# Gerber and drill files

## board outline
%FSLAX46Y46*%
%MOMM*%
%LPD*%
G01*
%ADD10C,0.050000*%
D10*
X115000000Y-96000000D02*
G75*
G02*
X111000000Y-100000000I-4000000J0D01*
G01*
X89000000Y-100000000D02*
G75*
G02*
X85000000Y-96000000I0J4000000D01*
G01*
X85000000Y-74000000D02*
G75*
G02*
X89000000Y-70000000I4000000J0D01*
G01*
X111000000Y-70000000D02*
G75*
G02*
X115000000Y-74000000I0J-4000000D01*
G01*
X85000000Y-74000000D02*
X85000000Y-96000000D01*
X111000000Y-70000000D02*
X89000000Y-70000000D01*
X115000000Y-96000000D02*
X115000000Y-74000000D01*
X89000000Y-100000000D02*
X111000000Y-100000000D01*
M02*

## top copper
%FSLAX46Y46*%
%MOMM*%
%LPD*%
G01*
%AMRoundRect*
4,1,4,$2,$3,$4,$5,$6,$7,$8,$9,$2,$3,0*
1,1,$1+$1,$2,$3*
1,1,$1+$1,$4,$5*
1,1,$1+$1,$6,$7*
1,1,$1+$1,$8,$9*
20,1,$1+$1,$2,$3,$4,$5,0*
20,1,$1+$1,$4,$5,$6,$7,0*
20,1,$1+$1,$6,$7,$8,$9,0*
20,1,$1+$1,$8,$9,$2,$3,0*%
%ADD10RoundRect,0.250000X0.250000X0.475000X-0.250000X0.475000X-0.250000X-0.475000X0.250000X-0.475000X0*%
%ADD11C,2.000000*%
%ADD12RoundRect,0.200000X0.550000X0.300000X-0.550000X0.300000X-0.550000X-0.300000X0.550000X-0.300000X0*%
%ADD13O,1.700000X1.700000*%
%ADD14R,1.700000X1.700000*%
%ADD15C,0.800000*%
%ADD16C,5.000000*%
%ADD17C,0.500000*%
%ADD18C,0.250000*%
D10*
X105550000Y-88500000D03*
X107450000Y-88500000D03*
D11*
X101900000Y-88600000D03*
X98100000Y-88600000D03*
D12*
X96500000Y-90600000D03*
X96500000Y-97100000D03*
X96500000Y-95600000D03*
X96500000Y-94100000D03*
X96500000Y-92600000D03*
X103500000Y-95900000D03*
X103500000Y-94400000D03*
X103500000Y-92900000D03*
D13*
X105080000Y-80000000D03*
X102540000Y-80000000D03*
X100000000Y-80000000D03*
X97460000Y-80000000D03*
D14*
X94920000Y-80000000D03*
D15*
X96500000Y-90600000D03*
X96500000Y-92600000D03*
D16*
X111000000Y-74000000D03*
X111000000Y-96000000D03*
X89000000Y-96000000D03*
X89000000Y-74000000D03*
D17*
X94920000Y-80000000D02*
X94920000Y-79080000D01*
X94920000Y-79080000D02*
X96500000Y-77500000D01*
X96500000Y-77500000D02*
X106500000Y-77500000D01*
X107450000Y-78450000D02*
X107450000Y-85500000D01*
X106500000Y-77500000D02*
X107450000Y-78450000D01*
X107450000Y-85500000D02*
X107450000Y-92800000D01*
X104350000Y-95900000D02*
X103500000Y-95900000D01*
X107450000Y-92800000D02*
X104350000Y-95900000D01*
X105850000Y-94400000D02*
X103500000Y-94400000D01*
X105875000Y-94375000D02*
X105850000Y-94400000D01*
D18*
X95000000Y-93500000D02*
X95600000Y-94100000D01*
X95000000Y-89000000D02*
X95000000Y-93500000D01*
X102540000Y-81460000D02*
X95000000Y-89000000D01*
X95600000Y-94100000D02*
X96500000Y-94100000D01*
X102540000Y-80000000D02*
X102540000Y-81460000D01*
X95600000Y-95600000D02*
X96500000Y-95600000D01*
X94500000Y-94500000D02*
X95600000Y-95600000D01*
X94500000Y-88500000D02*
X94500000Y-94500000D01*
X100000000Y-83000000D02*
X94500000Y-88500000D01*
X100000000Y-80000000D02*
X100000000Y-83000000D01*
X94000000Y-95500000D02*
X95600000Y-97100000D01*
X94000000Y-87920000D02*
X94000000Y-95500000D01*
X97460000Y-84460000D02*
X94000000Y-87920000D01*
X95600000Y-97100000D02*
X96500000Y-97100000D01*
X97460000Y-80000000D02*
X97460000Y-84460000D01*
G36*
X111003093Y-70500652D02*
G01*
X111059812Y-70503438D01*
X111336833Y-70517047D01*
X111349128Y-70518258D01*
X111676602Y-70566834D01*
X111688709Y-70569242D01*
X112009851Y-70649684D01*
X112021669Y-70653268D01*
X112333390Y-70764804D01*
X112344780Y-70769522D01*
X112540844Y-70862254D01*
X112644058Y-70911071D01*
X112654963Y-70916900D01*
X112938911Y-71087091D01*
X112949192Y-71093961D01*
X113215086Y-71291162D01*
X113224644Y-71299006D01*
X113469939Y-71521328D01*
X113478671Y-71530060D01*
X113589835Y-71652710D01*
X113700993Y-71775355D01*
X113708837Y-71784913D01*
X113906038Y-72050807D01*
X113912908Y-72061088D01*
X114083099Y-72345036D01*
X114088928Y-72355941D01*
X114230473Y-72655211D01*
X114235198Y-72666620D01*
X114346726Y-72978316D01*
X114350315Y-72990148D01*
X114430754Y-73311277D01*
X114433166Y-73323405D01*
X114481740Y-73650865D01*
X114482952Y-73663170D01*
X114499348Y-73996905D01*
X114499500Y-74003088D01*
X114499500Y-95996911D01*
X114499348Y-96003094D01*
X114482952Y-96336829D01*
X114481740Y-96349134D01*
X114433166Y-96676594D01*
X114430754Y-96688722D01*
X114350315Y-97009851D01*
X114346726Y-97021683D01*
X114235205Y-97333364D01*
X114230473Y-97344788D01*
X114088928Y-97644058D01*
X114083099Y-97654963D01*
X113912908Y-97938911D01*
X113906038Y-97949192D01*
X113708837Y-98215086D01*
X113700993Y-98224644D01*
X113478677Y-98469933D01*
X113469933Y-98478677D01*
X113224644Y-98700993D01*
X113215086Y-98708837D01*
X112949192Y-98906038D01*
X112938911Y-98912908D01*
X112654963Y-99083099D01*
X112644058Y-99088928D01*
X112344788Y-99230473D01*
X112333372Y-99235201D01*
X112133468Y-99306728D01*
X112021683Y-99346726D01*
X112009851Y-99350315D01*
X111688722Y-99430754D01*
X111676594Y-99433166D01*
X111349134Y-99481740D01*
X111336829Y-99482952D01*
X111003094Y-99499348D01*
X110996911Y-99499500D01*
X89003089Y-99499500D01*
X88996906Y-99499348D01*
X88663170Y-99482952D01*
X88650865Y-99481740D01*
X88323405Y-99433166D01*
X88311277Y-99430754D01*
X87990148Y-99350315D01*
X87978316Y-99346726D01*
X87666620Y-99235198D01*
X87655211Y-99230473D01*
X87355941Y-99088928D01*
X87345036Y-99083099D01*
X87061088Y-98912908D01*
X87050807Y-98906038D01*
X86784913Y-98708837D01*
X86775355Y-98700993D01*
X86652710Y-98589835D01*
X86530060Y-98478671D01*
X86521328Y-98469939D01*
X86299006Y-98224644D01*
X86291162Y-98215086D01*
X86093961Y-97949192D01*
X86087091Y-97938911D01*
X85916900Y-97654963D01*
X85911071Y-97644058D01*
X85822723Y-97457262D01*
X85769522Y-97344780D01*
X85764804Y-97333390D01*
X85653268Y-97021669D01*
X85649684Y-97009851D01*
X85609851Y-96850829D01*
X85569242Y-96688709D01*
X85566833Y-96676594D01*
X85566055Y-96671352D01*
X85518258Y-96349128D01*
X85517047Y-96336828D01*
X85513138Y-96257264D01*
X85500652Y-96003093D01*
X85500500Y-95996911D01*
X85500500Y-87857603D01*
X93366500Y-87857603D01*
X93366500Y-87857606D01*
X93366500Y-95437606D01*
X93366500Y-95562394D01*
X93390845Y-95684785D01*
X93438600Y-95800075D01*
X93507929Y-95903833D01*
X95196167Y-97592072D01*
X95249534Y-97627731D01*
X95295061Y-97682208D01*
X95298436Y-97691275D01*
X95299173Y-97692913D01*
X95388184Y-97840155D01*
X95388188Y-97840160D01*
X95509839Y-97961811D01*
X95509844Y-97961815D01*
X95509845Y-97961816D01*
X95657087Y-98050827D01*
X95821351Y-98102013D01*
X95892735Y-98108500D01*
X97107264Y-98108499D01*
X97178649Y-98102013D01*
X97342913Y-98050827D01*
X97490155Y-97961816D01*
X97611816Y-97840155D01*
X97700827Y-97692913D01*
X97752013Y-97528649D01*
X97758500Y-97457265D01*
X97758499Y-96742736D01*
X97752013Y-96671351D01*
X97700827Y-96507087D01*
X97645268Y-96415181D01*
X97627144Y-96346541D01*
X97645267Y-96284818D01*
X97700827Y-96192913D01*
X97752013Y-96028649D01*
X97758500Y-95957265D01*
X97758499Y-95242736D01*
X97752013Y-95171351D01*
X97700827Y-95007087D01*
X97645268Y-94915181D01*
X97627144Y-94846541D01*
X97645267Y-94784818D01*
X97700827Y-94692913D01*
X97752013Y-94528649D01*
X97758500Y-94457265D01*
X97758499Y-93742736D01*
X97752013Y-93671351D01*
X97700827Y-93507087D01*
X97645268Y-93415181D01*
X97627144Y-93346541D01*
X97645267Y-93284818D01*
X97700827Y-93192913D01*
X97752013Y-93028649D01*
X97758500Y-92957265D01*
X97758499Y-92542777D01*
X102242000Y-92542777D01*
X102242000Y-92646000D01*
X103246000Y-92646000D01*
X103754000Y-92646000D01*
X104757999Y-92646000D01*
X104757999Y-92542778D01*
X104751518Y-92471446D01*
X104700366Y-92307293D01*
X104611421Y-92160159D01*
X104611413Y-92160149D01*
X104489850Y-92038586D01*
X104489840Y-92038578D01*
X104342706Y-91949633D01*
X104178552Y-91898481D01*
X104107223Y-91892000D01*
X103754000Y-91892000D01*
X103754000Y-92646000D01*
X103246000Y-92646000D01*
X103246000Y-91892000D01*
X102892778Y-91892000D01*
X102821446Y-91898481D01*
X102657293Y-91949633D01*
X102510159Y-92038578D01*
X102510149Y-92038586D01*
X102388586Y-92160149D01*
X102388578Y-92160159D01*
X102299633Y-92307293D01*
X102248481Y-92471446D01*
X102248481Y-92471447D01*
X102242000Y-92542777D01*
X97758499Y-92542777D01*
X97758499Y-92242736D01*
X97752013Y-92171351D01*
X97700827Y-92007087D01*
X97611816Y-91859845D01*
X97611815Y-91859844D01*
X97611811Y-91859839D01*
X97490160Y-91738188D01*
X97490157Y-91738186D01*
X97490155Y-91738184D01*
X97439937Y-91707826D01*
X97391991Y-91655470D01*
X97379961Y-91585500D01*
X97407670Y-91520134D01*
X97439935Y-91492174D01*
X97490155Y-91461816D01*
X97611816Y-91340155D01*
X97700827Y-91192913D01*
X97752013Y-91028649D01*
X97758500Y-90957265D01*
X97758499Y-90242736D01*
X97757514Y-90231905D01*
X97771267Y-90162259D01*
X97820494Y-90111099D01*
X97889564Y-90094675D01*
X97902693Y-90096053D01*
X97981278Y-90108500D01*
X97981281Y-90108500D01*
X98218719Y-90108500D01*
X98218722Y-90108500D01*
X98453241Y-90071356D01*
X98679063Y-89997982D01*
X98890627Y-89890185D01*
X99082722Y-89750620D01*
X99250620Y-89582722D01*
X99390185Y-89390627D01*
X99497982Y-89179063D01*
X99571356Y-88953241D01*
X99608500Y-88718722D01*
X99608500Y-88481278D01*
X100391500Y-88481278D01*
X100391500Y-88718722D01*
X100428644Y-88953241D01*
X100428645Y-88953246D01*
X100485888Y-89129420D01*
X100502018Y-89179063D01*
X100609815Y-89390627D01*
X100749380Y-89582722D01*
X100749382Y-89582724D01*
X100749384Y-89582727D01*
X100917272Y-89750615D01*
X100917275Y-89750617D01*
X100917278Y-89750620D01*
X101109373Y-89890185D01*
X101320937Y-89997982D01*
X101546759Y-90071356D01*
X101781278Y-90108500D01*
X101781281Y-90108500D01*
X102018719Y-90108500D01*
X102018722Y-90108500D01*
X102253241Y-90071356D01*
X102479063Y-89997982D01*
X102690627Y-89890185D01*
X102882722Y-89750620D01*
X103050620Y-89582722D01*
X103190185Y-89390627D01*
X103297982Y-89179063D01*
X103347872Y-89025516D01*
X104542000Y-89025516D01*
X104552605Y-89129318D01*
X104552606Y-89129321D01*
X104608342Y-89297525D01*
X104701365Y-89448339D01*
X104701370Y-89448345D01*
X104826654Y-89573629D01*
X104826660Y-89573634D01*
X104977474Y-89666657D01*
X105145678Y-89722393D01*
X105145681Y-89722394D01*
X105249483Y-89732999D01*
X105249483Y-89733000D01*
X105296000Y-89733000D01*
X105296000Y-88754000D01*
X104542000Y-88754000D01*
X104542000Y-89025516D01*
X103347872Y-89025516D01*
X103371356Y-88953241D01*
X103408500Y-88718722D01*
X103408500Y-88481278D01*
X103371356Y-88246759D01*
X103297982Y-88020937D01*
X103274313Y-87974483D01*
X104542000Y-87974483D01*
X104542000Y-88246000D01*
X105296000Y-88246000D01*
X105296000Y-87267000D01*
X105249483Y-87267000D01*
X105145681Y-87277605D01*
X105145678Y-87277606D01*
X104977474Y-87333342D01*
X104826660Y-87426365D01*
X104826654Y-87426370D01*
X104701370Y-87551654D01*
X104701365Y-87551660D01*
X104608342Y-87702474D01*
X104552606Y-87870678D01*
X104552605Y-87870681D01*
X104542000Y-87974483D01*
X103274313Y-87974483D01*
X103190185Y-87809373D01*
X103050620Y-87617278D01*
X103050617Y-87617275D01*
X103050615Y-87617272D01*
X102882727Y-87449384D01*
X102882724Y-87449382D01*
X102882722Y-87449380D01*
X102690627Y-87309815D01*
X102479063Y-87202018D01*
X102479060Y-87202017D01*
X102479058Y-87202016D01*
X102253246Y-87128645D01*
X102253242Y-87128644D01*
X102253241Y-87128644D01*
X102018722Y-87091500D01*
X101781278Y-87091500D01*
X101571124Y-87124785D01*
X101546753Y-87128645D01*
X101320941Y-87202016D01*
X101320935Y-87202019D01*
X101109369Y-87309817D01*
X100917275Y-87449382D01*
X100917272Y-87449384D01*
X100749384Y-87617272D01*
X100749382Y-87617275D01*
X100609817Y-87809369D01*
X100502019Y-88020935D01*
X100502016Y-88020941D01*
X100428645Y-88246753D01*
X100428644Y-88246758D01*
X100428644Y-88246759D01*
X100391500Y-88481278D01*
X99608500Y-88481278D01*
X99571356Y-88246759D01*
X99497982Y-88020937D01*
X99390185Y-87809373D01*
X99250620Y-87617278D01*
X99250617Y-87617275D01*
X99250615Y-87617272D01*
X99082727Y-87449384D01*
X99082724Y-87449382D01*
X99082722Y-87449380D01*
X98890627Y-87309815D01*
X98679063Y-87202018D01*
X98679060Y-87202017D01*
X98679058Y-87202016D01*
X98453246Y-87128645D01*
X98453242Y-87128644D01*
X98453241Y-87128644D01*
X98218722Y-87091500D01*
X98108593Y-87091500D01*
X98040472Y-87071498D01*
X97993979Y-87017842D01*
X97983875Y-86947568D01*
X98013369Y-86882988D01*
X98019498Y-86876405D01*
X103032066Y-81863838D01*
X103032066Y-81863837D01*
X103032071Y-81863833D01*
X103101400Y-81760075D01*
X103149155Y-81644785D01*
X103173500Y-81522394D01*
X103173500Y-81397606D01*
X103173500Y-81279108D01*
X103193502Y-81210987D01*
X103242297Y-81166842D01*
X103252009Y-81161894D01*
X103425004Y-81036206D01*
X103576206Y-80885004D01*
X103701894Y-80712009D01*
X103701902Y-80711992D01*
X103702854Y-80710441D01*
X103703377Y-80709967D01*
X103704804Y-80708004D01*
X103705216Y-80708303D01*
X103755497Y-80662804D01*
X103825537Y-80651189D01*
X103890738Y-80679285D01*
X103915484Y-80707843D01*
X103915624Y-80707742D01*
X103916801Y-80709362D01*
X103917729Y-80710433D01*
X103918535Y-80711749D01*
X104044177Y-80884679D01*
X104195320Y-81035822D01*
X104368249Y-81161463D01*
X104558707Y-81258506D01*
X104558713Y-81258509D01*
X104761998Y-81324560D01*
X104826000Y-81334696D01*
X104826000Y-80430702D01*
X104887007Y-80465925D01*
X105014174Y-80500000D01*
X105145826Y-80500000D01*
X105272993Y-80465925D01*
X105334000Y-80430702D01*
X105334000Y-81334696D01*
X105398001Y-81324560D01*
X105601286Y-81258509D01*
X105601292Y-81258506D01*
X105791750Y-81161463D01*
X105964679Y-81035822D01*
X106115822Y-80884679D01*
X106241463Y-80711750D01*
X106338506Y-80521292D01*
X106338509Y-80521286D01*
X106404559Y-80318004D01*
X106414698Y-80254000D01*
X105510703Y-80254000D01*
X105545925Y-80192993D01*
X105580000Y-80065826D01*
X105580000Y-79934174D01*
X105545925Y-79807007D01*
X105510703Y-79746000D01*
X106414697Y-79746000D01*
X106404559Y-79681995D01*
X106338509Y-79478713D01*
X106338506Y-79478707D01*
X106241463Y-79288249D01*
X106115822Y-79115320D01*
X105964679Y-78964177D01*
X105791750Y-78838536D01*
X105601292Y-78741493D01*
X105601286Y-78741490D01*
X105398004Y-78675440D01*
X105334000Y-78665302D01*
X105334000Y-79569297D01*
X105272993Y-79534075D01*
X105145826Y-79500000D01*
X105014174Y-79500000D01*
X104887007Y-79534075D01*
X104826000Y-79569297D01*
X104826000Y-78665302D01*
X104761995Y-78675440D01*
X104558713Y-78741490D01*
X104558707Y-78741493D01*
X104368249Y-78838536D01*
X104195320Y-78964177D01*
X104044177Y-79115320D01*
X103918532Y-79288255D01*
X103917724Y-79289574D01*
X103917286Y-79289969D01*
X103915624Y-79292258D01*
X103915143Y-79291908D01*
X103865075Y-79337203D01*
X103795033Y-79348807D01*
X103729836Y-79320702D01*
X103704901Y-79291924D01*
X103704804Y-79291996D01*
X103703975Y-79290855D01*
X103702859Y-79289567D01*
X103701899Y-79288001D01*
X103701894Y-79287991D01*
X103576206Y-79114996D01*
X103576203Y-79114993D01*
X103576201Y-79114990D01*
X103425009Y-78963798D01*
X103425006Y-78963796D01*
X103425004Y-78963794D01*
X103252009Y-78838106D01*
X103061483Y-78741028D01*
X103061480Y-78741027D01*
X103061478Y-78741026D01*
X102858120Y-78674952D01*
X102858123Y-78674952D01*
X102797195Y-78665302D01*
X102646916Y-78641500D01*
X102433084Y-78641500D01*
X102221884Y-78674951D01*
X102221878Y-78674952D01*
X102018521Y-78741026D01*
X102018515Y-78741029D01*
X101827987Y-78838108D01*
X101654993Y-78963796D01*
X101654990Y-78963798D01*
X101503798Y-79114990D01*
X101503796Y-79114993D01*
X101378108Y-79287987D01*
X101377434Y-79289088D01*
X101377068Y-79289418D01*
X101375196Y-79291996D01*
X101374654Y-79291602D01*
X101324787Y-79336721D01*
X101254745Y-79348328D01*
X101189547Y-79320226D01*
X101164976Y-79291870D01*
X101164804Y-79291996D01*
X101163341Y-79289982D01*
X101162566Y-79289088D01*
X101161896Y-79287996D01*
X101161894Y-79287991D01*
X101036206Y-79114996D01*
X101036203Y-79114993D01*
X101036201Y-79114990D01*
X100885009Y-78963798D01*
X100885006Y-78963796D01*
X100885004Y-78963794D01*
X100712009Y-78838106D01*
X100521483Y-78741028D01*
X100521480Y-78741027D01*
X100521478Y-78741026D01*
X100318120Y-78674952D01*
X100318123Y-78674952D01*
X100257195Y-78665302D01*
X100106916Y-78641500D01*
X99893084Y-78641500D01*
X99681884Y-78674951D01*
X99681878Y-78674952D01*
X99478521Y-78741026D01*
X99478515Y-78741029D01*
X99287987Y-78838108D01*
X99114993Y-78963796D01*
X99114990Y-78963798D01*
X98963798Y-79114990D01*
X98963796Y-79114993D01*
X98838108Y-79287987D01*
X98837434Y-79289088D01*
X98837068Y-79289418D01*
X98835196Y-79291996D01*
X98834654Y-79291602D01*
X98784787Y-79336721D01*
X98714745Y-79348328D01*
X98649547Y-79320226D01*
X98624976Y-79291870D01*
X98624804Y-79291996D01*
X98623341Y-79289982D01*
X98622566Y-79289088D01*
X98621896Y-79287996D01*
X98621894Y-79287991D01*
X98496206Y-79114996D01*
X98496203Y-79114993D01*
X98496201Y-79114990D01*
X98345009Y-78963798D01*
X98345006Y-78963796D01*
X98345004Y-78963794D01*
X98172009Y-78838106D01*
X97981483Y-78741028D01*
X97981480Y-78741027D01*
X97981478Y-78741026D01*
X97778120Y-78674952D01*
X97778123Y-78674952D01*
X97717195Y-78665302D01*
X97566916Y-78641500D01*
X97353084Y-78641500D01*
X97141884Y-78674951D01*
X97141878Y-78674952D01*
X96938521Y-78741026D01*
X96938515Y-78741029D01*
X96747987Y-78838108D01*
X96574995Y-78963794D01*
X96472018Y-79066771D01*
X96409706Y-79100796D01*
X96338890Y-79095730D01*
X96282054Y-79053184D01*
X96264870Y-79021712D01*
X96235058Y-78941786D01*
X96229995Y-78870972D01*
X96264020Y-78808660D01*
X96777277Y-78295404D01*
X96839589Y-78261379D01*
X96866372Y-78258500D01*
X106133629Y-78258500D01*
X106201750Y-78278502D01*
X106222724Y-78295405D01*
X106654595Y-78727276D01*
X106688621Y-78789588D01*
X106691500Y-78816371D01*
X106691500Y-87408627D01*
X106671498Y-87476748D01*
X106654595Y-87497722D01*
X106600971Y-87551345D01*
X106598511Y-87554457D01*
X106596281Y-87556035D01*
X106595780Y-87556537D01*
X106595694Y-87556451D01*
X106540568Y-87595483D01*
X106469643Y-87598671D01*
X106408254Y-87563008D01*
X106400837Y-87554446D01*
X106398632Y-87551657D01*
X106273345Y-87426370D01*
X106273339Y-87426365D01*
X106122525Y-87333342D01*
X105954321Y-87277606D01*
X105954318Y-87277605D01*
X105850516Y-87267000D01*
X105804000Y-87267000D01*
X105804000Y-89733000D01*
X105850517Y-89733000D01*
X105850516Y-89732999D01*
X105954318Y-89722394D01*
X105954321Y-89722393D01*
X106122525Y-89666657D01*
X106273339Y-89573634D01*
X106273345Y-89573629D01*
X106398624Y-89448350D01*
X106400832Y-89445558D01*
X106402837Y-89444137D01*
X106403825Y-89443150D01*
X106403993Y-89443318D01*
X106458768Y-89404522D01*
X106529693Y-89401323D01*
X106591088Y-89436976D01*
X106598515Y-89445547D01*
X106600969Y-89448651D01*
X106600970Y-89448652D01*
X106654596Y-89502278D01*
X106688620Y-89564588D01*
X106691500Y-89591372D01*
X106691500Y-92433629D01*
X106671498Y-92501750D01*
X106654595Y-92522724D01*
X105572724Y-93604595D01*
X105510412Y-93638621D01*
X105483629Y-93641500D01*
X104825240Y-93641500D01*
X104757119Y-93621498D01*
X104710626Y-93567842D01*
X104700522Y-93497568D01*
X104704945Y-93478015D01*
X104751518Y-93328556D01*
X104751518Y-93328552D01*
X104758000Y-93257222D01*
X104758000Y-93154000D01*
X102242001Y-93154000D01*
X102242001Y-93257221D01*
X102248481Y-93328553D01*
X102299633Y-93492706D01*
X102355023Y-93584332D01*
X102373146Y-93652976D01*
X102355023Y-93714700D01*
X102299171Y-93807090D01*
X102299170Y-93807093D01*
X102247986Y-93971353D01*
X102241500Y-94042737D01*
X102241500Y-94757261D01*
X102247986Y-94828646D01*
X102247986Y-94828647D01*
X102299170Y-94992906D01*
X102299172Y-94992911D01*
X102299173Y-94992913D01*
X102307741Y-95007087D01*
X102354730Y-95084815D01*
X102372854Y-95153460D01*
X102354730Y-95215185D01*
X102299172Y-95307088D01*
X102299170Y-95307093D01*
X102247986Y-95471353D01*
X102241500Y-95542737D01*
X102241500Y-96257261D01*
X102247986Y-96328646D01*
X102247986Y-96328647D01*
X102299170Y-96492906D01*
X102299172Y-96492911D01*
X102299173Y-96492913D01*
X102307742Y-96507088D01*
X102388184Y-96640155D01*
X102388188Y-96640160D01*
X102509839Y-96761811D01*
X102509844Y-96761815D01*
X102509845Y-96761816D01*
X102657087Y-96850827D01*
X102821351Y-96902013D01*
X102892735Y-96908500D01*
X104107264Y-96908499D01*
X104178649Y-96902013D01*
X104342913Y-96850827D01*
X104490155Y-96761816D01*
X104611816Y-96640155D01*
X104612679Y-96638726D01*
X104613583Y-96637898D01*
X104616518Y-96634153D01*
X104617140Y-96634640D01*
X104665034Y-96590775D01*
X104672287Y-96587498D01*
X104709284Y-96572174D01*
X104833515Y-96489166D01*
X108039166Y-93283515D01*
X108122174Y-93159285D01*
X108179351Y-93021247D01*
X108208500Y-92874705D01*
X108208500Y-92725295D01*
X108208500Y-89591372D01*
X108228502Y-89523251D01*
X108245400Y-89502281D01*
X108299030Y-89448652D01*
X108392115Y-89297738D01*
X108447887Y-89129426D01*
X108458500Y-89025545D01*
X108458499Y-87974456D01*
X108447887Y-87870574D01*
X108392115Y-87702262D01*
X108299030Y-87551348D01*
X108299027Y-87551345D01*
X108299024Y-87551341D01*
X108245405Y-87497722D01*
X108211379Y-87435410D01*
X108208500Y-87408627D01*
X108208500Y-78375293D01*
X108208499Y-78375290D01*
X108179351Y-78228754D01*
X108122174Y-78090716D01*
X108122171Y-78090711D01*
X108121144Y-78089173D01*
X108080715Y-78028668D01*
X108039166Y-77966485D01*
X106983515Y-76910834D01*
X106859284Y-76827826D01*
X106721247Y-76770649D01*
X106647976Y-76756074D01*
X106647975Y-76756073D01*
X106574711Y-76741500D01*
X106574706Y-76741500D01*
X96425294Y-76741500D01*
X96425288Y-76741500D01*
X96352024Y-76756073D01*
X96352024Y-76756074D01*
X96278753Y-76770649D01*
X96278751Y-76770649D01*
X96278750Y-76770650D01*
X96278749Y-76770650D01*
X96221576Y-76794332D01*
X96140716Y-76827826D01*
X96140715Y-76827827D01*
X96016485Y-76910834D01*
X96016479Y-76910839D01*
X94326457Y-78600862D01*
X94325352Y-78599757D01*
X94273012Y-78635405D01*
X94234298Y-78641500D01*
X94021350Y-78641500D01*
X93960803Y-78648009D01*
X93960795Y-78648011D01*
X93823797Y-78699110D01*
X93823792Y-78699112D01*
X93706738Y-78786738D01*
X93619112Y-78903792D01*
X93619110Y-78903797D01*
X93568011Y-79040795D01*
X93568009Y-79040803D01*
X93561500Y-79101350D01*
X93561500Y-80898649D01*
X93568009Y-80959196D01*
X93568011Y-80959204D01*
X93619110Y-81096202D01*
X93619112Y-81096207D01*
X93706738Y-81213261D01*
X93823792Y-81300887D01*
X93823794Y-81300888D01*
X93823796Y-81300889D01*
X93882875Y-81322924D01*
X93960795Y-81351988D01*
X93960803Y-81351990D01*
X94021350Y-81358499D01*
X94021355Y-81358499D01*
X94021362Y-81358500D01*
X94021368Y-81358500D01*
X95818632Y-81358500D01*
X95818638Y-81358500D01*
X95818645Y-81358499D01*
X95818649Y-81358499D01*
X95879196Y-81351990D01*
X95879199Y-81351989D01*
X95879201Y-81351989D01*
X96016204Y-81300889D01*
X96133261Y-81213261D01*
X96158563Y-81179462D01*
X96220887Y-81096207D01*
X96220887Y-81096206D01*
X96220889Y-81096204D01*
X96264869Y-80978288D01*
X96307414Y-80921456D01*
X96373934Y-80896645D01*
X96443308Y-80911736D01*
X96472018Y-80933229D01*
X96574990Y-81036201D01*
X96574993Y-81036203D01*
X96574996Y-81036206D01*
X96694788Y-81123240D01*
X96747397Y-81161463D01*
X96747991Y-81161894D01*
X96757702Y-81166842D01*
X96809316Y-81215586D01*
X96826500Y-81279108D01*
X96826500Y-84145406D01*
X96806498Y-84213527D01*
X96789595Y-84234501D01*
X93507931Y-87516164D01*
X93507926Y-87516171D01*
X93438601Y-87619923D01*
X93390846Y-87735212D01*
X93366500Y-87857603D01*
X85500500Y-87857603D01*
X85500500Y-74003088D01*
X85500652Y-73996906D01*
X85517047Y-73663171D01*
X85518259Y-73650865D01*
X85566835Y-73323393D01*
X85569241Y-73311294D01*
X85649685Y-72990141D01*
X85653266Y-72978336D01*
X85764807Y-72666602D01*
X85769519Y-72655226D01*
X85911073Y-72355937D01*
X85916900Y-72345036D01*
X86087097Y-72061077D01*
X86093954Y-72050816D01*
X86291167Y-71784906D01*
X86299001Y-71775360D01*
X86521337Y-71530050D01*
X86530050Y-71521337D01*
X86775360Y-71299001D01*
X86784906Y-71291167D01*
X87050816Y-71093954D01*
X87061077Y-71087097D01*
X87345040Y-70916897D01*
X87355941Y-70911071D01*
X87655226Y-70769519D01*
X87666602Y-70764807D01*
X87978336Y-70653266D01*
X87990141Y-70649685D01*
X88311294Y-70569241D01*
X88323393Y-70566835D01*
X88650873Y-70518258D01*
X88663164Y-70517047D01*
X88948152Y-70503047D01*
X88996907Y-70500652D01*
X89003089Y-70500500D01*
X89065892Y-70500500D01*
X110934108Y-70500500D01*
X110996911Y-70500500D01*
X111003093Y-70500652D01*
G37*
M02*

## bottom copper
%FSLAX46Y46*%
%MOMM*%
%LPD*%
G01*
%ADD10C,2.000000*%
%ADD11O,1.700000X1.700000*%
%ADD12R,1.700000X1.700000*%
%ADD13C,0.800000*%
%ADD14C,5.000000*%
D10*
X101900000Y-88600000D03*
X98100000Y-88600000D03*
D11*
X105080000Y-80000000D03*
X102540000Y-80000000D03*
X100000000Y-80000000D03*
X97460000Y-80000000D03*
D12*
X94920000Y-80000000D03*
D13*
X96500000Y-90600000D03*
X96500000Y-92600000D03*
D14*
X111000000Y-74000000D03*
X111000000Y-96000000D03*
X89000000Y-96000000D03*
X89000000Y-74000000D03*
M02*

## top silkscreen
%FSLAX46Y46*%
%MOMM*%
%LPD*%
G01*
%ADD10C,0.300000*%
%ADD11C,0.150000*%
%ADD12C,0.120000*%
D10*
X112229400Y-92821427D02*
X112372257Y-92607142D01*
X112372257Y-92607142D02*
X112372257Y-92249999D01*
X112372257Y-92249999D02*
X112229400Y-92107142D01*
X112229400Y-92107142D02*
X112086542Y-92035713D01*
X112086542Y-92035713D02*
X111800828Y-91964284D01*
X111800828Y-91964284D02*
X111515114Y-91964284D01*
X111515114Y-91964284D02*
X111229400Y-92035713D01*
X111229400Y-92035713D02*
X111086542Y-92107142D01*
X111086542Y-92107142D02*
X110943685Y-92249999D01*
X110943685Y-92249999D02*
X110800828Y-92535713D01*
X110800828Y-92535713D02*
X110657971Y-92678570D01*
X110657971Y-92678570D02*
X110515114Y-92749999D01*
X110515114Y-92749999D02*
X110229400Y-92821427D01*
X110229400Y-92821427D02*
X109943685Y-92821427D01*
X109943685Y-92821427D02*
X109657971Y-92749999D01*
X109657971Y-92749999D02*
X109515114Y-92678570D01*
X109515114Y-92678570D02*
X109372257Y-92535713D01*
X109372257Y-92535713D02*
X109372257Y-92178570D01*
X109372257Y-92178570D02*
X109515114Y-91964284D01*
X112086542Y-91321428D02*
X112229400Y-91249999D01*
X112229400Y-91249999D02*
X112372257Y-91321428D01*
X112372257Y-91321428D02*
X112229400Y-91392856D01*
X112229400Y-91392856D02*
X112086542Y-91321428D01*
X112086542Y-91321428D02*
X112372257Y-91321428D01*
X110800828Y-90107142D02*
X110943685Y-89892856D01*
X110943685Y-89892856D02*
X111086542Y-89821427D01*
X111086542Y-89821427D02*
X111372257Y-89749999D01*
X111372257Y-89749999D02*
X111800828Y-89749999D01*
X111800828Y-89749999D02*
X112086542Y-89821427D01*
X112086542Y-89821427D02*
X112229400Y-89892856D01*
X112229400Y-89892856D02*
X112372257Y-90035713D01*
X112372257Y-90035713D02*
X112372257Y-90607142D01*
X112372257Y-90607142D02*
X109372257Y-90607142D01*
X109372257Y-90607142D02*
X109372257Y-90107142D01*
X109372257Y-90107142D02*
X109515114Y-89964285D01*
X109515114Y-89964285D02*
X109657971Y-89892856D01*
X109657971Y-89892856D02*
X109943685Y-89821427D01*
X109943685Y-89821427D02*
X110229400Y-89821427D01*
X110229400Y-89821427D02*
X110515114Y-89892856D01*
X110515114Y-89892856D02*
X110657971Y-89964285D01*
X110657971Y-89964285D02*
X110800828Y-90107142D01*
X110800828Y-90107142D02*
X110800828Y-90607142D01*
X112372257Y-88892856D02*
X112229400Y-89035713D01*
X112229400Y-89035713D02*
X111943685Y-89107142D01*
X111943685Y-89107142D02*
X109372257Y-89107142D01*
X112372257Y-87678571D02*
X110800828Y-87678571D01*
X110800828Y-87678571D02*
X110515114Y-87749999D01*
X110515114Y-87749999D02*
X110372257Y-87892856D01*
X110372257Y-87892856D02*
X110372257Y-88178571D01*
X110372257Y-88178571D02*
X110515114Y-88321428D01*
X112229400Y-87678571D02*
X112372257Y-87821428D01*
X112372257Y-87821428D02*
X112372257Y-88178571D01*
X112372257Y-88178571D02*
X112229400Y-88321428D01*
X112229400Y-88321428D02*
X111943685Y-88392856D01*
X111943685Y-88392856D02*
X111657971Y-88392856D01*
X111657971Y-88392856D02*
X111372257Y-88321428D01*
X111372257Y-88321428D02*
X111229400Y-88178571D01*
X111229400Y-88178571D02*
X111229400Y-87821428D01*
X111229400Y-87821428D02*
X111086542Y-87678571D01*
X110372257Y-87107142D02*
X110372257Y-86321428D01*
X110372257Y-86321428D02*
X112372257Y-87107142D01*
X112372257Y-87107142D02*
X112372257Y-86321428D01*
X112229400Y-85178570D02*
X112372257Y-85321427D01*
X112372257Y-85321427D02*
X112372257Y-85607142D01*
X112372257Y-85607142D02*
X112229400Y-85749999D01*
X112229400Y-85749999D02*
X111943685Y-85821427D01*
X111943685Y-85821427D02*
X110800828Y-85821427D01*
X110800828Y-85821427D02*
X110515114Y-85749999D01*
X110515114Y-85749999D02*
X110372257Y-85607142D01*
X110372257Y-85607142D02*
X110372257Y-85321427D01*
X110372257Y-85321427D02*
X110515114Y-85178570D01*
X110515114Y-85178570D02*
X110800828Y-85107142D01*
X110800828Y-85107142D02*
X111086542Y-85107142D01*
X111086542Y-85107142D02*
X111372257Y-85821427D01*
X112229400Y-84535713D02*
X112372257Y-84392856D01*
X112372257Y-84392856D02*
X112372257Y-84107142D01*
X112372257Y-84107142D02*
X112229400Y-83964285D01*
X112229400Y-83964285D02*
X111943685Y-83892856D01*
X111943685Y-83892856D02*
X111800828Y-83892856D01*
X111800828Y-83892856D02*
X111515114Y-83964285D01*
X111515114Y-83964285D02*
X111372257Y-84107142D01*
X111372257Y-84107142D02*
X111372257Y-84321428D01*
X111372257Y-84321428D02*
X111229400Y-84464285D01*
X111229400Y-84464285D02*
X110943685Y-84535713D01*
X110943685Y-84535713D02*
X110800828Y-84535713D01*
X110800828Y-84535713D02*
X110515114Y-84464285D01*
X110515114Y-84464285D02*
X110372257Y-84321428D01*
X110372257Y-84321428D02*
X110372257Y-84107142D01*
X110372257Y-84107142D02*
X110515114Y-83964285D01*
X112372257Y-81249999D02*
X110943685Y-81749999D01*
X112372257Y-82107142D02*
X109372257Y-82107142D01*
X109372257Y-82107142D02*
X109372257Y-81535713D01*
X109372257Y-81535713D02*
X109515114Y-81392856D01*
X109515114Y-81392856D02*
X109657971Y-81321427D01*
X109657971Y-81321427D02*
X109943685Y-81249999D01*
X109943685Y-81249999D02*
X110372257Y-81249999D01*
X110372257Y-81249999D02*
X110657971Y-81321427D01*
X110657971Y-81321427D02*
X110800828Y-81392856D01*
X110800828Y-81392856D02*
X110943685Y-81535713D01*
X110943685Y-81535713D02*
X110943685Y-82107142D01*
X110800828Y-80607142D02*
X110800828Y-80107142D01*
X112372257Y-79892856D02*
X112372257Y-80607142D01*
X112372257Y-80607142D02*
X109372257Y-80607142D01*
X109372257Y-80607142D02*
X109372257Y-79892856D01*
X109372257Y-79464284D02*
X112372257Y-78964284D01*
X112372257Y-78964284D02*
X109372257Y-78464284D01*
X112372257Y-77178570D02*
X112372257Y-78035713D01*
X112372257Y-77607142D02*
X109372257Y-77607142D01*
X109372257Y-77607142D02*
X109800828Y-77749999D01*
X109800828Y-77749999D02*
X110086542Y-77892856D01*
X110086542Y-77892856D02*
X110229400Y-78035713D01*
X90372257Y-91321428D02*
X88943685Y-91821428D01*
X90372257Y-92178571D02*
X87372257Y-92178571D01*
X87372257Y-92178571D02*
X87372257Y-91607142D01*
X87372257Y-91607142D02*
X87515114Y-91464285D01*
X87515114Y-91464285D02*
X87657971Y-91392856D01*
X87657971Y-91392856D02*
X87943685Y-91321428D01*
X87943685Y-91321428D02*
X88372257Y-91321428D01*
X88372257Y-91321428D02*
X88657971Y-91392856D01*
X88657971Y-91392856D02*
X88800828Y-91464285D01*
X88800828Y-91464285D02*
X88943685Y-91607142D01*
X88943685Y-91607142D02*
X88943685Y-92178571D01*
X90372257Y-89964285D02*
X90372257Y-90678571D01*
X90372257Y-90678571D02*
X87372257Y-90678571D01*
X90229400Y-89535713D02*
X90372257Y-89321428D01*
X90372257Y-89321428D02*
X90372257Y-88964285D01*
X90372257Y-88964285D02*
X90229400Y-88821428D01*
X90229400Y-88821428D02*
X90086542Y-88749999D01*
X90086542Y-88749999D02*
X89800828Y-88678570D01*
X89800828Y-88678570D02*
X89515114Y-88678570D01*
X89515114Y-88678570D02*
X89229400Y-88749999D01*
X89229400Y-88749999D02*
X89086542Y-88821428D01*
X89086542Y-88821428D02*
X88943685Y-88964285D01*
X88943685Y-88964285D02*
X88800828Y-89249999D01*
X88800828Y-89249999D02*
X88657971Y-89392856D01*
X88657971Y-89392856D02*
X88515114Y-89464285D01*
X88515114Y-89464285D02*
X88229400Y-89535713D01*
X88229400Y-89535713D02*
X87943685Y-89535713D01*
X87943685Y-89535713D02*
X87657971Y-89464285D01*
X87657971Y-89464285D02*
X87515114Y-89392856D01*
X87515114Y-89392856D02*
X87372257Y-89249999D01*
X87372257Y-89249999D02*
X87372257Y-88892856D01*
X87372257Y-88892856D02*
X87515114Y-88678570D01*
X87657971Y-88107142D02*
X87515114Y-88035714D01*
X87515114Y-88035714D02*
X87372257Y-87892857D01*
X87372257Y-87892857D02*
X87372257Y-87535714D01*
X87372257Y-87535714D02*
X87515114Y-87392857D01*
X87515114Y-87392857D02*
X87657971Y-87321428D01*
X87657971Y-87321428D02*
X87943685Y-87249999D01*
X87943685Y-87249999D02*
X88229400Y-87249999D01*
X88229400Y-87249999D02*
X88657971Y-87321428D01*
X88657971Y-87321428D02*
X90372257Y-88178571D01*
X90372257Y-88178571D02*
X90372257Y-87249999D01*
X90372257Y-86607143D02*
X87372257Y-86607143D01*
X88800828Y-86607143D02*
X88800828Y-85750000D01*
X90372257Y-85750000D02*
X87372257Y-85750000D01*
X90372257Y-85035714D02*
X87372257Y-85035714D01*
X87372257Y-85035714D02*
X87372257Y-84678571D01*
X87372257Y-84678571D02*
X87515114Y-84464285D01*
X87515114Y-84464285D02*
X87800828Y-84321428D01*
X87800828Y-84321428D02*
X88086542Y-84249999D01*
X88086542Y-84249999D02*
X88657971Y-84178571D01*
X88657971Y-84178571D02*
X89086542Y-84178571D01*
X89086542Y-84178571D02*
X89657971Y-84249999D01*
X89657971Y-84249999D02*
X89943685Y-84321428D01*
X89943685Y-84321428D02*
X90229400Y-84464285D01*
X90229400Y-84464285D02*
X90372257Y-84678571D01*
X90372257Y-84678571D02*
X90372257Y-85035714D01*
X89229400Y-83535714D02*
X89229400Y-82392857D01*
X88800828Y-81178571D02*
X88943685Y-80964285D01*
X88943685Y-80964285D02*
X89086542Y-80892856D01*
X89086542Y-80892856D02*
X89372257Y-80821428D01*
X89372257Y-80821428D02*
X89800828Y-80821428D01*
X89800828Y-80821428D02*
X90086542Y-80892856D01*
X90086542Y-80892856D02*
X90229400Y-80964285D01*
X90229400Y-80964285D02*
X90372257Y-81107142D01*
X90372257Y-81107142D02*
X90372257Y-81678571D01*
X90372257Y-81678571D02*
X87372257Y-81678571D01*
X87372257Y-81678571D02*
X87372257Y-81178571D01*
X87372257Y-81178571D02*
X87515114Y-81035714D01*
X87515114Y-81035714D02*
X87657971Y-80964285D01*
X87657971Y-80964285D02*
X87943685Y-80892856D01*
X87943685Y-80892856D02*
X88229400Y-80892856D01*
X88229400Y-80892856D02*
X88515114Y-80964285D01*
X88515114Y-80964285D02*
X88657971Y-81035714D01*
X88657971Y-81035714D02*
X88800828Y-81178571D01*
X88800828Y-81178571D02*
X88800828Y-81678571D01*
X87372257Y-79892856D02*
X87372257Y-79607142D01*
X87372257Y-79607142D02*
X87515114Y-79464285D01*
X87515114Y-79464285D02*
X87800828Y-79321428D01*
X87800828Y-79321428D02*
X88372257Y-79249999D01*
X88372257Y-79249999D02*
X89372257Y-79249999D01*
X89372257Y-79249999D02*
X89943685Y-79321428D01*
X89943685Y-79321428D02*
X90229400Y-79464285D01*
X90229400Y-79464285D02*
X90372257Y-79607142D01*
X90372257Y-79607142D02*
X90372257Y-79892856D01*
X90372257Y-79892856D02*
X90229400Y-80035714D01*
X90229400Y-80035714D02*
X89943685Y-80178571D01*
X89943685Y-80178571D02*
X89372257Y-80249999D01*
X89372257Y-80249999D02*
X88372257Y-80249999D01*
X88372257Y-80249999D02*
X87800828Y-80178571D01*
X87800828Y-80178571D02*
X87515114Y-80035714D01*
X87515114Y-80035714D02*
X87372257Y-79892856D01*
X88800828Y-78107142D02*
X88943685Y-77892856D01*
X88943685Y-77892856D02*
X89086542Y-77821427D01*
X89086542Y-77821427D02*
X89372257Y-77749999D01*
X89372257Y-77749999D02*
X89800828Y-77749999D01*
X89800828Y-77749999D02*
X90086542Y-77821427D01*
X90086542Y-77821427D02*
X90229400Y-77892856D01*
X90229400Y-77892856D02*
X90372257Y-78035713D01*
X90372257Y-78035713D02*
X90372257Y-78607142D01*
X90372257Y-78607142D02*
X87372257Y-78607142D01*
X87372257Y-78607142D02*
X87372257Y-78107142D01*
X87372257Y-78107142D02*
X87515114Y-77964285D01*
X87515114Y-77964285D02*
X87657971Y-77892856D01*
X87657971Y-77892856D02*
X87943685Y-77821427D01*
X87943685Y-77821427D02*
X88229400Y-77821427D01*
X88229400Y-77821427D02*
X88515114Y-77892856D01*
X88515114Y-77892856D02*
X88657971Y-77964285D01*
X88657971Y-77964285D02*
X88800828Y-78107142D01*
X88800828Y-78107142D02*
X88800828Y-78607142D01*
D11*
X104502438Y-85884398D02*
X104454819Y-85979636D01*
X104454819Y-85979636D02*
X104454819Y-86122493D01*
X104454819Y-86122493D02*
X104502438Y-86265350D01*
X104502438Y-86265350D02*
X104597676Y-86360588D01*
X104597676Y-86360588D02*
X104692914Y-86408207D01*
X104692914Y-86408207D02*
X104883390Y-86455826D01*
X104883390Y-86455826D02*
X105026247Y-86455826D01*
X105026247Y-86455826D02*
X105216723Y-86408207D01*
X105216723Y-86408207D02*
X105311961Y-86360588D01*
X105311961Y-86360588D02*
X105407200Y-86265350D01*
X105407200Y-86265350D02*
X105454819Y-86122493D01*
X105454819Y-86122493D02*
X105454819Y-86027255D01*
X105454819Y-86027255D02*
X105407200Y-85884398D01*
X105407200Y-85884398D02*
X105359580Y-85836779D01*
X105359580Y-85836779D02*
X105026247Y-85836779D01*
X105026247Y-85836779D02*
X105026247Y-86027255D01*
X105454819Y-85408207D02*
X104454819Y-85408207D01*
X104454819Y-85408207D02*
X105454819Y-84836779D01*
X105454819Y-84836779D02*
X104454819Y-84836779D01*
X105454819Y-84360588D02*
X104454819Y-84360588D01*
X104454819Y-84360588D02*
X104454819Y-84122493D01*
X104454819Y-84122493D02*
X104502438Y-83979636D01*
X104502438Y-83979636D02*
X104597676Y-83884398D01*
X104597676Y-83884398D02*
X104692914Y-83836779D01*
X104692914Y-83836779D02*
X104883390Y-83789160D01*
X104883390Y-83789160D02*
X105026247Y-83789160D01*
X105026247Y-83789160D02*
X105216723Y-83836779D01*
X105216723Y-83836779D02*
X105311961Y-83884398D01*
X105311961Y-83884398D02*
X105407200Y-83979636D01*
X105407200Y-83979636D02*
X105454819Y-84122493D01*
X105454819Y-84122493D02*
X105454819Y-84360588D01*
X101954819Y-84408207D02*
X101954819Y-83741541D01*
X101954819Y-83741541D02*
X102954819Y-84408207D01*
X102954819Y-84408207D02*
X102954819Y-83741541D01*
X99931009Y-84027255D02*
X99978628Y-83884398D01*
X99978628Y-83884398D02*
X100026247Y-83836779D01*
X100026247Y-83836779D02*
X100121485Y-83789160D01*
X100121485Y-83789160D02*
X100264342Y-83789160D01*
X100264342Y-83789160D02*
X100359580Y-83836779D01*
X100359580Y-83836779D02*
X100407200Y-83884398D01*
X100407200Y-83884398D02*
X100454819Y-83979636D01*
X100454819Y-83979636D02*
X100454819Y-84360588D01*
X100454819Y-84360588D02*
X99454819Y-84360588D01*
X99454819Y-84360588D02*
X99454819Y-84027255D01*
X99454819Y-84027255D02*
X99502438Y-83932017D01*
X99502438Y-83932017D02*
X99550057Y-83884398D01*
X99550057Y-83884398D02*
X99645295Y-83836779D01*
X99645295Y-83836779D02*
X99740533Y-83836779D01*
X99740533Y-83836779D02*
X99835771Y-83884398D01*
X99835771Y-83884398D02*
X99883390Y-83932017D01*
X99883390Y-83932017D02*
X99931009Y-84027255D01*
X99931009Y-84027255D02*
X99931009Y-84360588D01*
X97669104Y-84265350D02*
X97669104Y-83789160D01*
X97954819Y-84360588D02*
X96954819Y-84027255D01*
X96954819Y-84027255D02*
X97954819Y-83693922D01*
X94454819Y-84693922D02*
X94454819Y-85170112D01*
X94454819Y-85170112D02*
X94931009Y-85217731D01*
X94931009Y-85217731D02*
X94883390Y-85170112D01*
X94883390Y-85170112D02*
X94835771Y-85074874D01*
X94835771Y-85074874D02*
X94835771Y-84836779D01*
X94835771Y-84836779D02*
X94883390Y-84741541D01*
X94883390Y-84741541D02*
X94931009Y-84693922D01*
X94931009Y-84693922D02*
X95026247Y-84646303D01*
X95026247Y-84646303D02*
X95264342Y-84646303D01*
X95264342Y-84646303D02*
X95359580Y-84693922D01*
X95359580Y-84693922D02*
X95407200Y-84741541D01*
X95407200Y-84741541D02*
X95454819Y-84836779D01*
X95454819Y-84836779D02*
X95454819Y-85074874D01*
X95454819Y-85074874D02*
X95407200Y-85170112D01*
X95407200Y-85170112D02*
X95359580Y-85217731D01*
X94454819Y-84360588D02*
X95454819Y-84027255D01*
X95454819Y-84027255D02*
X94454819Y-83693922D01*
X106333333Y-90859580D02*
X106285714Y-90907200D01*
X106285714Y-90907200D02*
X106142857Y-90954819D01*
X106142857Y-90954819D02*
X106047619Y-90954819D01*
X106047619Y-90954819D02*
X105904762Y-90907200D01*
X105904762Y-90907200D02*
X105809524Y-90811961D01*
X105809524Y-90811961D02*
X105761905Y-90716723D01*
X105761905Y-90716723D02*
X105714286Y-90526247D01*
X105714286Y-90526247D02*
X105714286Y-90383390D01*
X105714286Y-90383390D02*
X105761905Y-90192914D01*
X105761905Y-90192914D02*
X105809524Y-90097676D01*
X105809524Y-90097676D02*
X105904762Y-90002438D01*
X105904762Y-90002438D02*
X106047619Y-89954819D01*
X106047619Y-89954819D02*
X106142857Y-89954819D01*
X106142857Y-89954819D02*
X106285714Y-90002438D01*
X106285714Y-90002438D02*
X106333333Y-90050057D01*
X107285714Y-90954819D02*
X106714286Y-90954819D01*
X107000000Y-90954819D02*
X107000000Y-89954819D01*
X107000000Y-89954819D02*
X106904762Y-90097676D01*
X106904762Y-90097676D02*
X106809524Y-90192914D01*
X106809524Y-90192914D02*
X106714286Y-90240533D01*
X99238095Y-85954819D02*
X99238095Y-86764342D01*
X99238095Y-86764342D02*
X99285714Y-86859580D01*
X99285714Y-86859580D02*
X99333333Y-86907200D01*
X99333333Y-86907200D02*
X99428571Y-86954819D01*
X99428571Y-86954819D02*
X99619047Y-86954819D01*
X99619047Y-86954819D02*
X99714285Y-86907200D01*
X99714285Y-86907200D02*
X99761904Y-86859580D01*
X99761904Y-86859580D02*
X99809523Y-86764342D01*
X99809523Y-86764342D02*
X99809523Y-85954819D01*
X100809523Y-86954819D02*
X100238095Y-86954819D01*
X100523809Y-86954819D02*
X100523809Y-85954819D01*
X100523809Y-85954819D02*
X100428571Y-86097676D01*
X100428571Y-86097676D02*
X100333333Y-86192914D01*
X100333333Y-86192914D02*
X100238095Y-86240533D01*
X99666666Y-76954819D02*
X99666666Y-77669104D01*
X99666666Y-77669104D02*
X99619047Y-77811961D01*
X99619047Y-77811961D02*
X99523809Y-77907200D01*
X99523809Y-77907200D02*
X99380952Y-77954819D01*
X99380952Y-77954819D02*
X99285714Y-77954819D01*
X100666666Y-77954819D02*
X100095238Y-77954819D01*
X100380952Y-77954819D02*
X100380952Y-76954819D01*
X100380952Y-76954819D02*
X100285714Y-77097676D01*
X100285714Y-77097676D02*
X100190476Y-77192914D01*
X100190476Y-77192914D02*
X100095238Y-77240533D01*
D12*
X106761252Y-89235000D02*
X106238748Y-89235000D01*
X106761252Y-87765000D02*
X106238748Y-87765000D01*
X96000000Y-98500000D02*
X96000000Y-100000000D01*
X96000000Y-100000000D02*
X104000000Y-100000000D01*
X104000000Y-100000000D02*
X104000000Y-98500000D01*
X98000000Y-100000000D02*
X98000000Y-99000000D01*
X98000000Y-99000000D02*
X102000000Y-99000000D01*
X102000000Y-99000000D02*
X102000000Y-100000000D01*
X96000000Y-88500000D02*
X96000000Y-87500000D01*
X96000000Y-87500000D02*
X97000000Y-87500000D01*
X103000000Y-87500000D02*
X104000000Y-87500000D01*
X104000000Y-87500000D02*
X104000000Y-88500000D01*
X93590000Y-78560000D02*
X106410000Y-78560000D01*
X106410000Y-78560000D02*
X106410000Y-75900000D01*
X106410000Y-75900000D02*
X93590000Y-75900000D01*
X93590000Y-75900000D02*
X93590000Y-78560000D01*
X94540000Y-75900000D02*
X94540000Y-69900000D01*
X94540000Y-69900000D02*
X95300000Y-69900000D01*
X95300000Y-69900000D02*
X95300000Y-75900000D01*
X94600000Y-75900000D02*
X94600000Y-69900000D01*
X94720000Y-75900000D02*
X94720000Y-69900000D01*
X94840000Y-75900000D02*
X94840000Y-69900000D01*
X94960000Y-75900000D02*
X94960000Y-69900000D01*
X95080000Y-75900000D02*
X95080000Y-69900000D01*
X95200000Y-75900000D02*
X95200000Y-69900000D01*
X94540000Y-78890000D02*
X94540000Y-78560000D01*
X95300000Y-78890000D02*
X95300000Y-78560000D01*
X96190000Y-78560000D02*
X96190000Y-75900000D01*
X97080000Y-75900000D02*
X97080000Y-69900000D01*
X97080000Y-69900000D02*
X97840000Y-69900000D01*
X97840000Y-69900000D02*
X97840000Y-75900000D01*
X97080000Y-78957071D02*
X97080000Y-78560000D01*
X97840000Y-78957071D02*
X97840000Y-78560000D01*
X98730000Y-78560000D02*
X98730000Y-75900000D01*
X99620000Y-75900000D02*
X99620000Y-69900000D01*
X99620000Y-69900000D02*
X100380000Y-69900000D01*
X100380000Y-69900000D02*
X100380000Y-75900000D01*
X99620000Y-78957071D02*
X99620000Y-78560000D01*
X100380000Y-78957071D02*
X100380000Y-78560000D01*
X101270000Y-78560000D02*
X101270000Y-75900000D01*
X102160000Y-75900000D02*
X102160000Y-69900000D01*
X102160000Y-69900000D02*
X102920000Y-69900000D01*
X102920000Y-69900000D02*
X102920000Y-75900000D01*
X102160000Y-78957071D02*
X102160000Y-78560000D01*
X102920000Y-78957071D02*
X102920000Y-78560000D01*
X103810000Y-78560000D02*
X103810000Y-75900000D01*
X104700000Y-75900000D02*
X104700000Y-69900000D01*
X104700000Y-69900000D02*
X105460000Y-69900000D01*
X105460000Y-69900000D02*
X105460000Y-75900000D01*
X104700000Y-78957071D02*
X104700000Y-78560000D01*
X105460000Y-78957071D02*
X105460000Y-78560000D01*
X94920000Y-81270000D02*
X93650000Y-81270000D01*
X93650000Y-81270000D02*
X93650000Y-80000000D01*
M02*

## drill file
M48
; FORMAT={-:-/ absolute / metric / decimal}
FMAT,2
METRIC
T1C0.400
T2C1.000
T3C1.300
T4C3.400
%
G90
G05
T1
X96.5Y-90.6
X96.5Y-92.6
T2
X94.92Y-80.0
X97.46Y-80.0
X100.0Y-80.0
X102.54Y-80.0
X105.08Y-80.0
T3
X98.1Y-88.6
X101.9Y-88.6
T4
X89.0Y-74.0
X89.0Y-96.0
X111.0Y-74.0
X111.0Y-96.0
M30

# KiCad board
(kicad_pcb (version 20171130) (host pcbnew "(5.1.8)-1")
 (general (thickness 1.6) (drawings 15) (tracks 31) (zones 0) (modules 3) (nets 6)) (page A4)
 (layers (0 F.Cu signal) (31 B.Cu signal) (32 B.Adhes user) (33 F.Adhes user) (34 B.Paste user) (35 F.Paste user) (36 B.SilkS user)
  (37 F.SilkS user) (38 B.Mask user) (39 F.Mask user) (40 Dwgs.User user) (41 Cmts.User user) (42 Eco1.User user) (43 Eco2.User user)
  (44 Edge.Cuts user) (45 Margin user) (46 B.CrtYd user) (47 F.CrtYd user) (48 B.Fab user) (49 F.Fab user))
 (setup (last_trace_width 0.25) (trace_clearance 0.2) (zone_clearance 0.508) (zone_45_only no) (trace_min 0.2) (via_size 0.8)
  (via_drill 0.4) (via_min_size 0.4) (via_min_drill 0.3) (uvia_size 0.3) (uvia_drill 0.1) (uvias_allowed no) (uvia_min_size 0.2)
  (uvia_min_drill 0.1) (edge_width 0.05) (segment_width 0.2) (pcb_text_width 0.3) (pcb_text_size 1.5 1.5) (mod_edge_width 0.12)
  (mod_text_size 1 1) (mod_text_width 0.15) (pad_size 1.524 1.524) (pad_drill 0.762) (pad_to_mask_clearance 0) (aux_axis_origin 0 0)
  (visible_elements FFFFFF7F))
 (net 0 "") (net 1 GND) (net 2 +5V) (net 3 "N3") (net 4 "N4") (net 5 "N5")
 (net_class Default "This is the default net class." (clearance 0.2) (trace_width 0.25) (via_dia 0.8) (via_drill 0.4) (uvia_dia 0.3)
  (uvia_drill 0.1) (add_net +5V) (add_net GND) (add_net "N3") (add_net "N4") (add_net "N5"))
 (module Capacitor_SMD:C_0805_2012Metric (layer F.Cu) (at 106.5 88.5 180)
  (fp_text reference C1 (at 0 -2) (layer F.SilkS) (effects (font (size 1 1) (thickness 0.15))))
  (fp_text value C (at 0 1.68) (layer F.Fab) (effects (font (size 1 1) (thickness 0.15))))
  (fp_line (start -0.261252 -0.735) (end 0.261252 -0.735) (layer F.SilkS) (width 0.12))
  (fp_line (start -0.261252 0.735) (end 0.261252 0.735) (layer F.SilkS) (width 0.12))
  (pad 2 smd roundrect (at 0.95 0 180) (size 1 1.45) (layers F.Cu F.Paste F.Mask) (roundrect_rratio 0.25) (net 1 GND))
  (pad 1 smd roundrect (at -0.95 0 180) (size 1 1.45) (layers F.Cu F.Paste F.Mask) (roundrect_rratio 0.25) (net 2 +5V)))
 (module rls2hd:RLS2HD (layer F.Cu) (at 100 100)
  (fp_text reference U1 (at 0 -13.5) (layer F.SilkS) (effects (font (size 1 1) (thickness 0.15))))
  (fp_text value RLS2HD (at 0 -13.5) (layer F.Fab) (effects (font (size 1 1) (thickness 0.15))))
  (fp_line (start -4 -1.5) (end -4 0) (layer F.SilkS) (width 0.12))
  (fp_line (start -4 0) (end 4 0) (layer F.SilkS) (width 0.12))
  (fp_line (start 4 0) (end 4 -1.5) (layer F.SilkS) (width 0.12))
  (fp_line (start -2 0) (end -2 -1) (layer F.SilkS) (width 0.12))
  (fp_line (start -2 -1) (end 2 -1) (layer F.SilkS) (width 0.12))
  (fp_line (start 2 -1) (end 2 0) (layer F.SilkS) (width 0.12))
  (fp_line (start -4 -11.5) (end -4 -12.5) (layer F.SilkS) (width 0.12))
  (fp_line (start -4 -12.5) (end -3 -12.5) (layer F.SilkS) (width 0.12))
  (fp_line (start 3 -12.5) (end 4 -12.5) (layer F.SilkS) (width 0.12))
  (fp_line (start 4 -12.5) (end 4 -11.5) (layer F.SilkS) (width 0.12))
  (pad "" thru_hole circle (at 1.9 -11.4) (size 2 2) (drill 1.3) (layers *.Cu *.Mask))
  (pad "" thru_hole circle (at -1.9 -11.4) (size 2 2) (drill 1.3) (layers *.Cu *.Mask))
  (pad 4 smd roundrect (at -3.5 -9.4 180) (size 1.5 1) (layers F.Cu F.Paste F.Mask) (roundrect_rratio 0.2))
  (pad 8 smd roundrect (at -3.5 -2.9 180) (size 1.5 1) (layers F.Cu F.Paste F.Mask) (roundrect_rratio 0.2) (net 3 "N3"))
  (pad 7 smd roundrect (at -3.5 -4.4 180) (size 1.5 1) (layers F.Cu F.Paste F.Mask) (roundrect_rratio 0.2) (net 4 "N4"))
  (pad 6 smd roundrect (at -3.5 -5.9 180) (size 1.5 1) (layers F.Cu F.Paste F.Mask) (roundrect_rratio 0.2) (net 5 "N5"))
  (pad 5 smd roundrect (at -3.5 -7.4 180) (size 1.5 1) (layers F.Cu F.Paste F.Mask) (roundrect_rratio 0.2))
  (pad 1 smd roundrect (at 3.5 -4.1 180) (size 1.5 1) (layers F.Cu F.Paste F.Mask) (roundrect_rratio 0.2) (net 2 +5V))
  (pad 2 smd roundrect (at 3.5 -5.6 180) (size 1.5 1) (layers F.Cu F.Paste F.Mask) (roundrect_rratio 0.2) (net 2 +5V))
  (pad 3 smd roundrect (at 3.5 -7.1 180) (size 1.5 1) (layers F.Cu F.Paste F.Mask) (roundrect_rratio 0.2) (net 1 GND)))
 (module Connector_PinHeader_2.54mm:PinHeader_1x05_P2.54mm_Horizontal (layer F.Cu) (at 94.92 80 90)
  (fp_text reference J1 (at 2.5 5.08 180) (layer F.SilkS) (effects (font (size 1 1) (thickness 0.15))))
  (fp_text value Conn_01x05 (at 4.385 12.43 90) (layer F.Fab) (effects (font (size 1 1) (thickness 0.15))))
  (fp_line (start 1.44 -1.33) (end 1.44 11.49) (layer F.SilkS) (width 0.12))
  (fp_line (start 1.44 11.49) (end 4.1 11.49) (layer F.SilkS) (width 0.12))
  (fp_line (start 4.1 11.49) (end 4.1 -1.33) (layer F.SilkS) (width 0.12))
  (fp_line (start 4.1 -1.33) (end 1.44 -1.33) (layer F.SilkS) (width 0.12))
  (fp_line (start 4.1 -0.38) (end 10.1 -0.38) (layer F.SilkS) (width 0.12))
  (fp_line (start 10.1 -0.38) (end 10.1 0.38) (layer F.SilkS) (width 0.12))
  (fp_line (start 10.1 0.38) (end 4.1 0.38) (layer F.SilkS) (width 0.12))
  (fp_line (start 4.1 -0.32) (end 10.1 -0.32) (layer F.SilkS) (width 0.12))
  (fp_line (start 4.1 -0.2) (end 10.1 -0.2) (layer F.SilkS) (width 0.12))
  (fp_line (start 4.1 -0.08) (end 10.1 -0.08) (layer F.SilkS) (width 0.12))
  (fp_line (start 4.1 0.04) (end 10.1 0.04) (layer F.SilkS) (width 0.12))
  (fp_line (start 4.1 0.16) (end 10.1 0.16) (layer F.SilkS) (width 0.12))
  (fp_line (start 4.1 0.28) (end 10.1 0.28) (layer F.SilkS) (width 0.12))
  (fp_line (start 1.11 -0.38) (end 1.44 -0.38) (layer F.SilkS) (width 0.12))
  (fp_line (start 1.11 0.38) (end 1.44 0.38) (layer F.SilkS) (width 0.12))
  (fp_line (start 1.44 1.27) (end 4.1 1.27) (layer F.SilkS) (width 0.12))
  (fp_line (start 4.1 2.16) (end 10.1 2.16) (layer F.SilkS) (width 0.12))
  (fp_line (start 10.1 2.16) (end 10.1 2.92) (layer F.SilkS) (width 0.12))
  (fp_line (start 10.1 2.92) (end 4.1 2.92) (layer F.SilkS) (width 0.12))
  (fp_line (start 1.042929 2.16) (end 1.44 2.16) (layer F.SilkS) (width 0.12))
  (fp_line (start 1.042929 2.92) (end 1.44 2.92) (layer F.SilkS) (width 0.12))
  (fp_line (start 1.44 3.81) (end 4.1 3.81) (layer F.SilkS) (width 0.12))
  (fp_line (start 4.1 4.7) (end 10.1 4.7) (layer F.SilkS) (width 0.12))
  (fp_line (start 10.1 4.7) (end 10.1 5.46) (layer F.SilkS) (width 0.12))
  (fp_line (start 10.1 5.46) (end 4.1 5.46) (layer F.SilkS) (width 0.12))
  (fp_line (start 1.042929 4.7) (end 1.44 4.7) (layer F.SilkS) (width 0.12))
  (fp_line (start 1.042929 5.46) (end 1.44 5.46) (layer F.SilkS) (width 0.12))
  (fp_line (start 1.44 6.35) (end 4.1 6.35) (layer F.SilkS) (width 0.12))
  (fp_line (start 4.1 7.24) (end 10.1 7.24) (layer F.SilkS) (width 0.12))
  (fp_line (start 10.1 7.24) (end 10.1 8) (layer F.SilkS) (width 0.12))
  (fp_line (start 10.1 8) (end 4.1 8) (layer F.SilkS) (width 0.12))
  (fp_line (start 1.042929 7.24) (end 1.44 7.24) (layer F.SilkS) (width 0.12))
  (fp_line (start 1.042929 8) (end 1.44 8) (layer F.SilkS) (width 0.12))
  (fp_line (start 1.44 8.89) (end 4.1 8.89) (layer F.SilkS) (width 0.12))
  (fp_line (start 4.1 9.78) (end 10.1 9.78) (layer F.SilkS) (width 0.12))
  (fp_line (start 10.1 9.78) (end 10.1 10.54) (layer F.SilkS) (width 0.12))
  (fp_line (start 10.1 10.54) (end 4.1 10.54) (layer F.SilkS) (width 0.12))
  (fp_line (start 1.042929 9.78) (end 1.44 9.78) (layer F.SilkS) (width 0.12))
  (fp_line (start 1.042929 10.54) (end 1.44 10.54) (layer F.SilkS) (width 0.12))
  (fp_line (start -1.27 0) (end -1.27 -1.27) (layer F.SilkS) (width 0.12))
  (fp_line (start -1.27 -1.27) (end 0 -1.27) (layer F.SilkS) (width 0.12))
  (pad 5 thru_hole oval (at 0 10.16 90) (size 1.7 1.7) (drill 1) (layers *.Cu *.Mask) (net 1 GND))
  (pad 4 thru_hole oval (at 0 7.62 90) (size 1.7 1.7) (drill 1) (layers *.Cu *.Mask) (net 5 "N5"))
  (pad 3 thru_hole oval (at 0 5.08 90) (size 1.7 1.7) (drill 1) (layers *.Cu *.Mask) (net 4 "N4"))
  (pad 2 thru_hole oval (at 0 2.54 90) (size 1.7 1.7) (drill 1) (layers *.Cu *.Mask) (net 3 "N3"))
  (pad 1 thru_hole rect (at 0 0 90) (size 1.7 1.7) (drill 1) (layers *.Cu *.Mask) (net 2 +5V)))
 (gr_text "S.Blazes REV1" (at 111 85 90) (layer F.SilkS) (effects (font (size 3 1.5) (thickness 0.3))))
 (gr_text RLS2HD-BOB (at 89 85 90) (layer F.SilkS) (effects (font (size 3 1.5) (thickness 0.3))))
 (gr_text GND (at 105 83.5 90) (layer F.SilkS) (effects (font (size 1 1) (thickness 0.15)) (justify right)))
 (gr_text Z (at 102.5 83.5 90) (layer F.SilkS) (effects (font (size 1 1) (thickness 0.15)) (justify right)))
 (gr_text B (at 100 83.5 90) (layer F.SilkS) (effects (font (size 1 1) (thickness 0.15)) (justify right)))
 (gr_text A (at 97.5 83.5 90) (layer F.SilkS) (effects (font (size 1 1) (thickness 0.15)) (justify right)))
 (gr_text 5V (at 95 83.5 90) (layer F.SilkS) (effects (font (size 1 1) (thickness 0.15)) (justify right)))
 (gr_arc (start 111 96) (end 111 100) (angle -90) (layer Edge.Cuts) (width 0.05))
 (gr_arc (start 89 96) (end 85 96) (angle -90) (layer Edge.Cuts) (width 0.05))
 (gr_arc (start 89 74) (end 89 70) (angle -90) (layer Edge.Cuts) (width 0.05))
 (gr_arc (start 111 74) (end 115 74) (angle -90) (layer Edge.Cuts) (width 0.05))
 (gr_line (start 85 74) (end 85 96) (layer Edge.Cuts) (width 0.05))
 (gr_line (start 111 70) (end 89 70) (layer Edge.Cuts) (width 0.05))
 (gr_line (start 115 96) (end 115 74) (layer Edge.Cuts) (width 0.05))
 (gr_line (start 89 100) (end 111 100) (layer Edge.Cuts) (width 0.05))
 (via (at 96.5 90.6) (size 0.8) (drill 0.4) (layers F.Cu B.Cu) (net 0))
 (via (at 96.5 92.6) (size 0.8) (drill 0.4) (layers F.Cu B.Cu) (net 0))
 (via (at 111 74) (size 5) (drill 3.4) (layers F.Cu B.Cu) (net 1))
 (via (at 111 96) (size 5) (drill 3.4) (layers F.Cu B.Cu) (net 1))
 (via (at 89 96) (size 5) (drill 3.4) (layers F.Cu B.Cu) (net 1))
 (via (at 89 74) (size 5) (drill 3.4) (layers F.Cu B.Cu) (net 1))
 (segment (start 94.92 80) (end 94.92 79.08) (width 0.5) (layer F.Cu) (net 2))
 (segment (start 94.92 79.08) (end 96.5 77.5) (width 0.5) (layer F.Cu) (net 2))
 (segment (start 96.5 77.5) (end 106.5 77.5) (width 0.5) (layer F.Cu) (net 2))
 (segment (start 107.45 78.45) (end 107.45 85.5) (width 0.5) (layer F.Cu) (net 2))
 (segment (start 106.5 77.5) (end 107.45 78.45) (width 0.5) (layer F.Cu) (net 2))
 (segment (start 107.45 85.5) (end 107.45 92.8) (width 0.5) (layer F.Cu) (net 2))
 (segment (start 104.35 95.9) (end 103.5 95.9) (width 0.5) (layer F.Cu) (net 2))
 (segment (start 107.45 92.8) (end 104.35 95.9) (width 0.5) (layer F.Cu) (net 2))
 (segment (start 105.85 94.4) (end 103.5 94.4) (width 0.5) (layer F.Cu) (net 2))
 (segment (start 105.875 94.375) (end 105.85 94.4) (width 0.5) (layer F.Cu) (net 2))
 (segment (start 95 93.5) (end 95.6 94.1) (width 0.25) (layer F.Cu) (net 5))
 (segment (start 95 89) (end 95 93.5) (width 0.25) (layer F.Cu) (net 5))
 (segment (start 102.54 81.46) (end 95 89) (width 0.25) (layer F.Cu) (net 5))
 (segment (start 95.6 94.1) (end 96.5 94.1) (width 0.25) (layer F.Cu) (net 5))
 (segment (start 102.54 80) (end 102.54 81.46) (width 0.25) (layer F.Cu) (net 5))
 (segment (start 95.6 95.6) (end 96.5 95.6) (width 0.25) (layer F.Cu) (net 4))
 (segment (start 94.5 94.5) (end 95.6 95.6) (width 0.25) (layer F.Cu) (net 4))
 (segment (start 94.5 88.5) (end 94.5 94.5) (width 0.25) (layer F.Cu) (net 4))
 (segment (start 100 83) (end 94.5 88.5) (width 0.25) (layer F.Cu) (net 4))
 (segment (start 100 80) (end 100 83) (width 0.25) (layer F.Cu) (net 4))
 (segment (start 94 95.5) (end 95.6 97.1) (width 0.25) (layer F.Cu) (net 3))
 (segment (start 94 87.92) (end 94 95.5) (width 0.25) (layer F.Cu) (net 3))
 (segment (start 97.46 84.46) (end 94 87.92) (width 0.25) (layer F.Cu) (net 3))
 (segment (start 95.6 97.1) (end 96.5 97.1) (width 0.25) (layer F.Cu) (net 3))
 (segment (start 97.46 80) (end 97.46 84.46) (width 0.25) (layer F.Cu) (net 3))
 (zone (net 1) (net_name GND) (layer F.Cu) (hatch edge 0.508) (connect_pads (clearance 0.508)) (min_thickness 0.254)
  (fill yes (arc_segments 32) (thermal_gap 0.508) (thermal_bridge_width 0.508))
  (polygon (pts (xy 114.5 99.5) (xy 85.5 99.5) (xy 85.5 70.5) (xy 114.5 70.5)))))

